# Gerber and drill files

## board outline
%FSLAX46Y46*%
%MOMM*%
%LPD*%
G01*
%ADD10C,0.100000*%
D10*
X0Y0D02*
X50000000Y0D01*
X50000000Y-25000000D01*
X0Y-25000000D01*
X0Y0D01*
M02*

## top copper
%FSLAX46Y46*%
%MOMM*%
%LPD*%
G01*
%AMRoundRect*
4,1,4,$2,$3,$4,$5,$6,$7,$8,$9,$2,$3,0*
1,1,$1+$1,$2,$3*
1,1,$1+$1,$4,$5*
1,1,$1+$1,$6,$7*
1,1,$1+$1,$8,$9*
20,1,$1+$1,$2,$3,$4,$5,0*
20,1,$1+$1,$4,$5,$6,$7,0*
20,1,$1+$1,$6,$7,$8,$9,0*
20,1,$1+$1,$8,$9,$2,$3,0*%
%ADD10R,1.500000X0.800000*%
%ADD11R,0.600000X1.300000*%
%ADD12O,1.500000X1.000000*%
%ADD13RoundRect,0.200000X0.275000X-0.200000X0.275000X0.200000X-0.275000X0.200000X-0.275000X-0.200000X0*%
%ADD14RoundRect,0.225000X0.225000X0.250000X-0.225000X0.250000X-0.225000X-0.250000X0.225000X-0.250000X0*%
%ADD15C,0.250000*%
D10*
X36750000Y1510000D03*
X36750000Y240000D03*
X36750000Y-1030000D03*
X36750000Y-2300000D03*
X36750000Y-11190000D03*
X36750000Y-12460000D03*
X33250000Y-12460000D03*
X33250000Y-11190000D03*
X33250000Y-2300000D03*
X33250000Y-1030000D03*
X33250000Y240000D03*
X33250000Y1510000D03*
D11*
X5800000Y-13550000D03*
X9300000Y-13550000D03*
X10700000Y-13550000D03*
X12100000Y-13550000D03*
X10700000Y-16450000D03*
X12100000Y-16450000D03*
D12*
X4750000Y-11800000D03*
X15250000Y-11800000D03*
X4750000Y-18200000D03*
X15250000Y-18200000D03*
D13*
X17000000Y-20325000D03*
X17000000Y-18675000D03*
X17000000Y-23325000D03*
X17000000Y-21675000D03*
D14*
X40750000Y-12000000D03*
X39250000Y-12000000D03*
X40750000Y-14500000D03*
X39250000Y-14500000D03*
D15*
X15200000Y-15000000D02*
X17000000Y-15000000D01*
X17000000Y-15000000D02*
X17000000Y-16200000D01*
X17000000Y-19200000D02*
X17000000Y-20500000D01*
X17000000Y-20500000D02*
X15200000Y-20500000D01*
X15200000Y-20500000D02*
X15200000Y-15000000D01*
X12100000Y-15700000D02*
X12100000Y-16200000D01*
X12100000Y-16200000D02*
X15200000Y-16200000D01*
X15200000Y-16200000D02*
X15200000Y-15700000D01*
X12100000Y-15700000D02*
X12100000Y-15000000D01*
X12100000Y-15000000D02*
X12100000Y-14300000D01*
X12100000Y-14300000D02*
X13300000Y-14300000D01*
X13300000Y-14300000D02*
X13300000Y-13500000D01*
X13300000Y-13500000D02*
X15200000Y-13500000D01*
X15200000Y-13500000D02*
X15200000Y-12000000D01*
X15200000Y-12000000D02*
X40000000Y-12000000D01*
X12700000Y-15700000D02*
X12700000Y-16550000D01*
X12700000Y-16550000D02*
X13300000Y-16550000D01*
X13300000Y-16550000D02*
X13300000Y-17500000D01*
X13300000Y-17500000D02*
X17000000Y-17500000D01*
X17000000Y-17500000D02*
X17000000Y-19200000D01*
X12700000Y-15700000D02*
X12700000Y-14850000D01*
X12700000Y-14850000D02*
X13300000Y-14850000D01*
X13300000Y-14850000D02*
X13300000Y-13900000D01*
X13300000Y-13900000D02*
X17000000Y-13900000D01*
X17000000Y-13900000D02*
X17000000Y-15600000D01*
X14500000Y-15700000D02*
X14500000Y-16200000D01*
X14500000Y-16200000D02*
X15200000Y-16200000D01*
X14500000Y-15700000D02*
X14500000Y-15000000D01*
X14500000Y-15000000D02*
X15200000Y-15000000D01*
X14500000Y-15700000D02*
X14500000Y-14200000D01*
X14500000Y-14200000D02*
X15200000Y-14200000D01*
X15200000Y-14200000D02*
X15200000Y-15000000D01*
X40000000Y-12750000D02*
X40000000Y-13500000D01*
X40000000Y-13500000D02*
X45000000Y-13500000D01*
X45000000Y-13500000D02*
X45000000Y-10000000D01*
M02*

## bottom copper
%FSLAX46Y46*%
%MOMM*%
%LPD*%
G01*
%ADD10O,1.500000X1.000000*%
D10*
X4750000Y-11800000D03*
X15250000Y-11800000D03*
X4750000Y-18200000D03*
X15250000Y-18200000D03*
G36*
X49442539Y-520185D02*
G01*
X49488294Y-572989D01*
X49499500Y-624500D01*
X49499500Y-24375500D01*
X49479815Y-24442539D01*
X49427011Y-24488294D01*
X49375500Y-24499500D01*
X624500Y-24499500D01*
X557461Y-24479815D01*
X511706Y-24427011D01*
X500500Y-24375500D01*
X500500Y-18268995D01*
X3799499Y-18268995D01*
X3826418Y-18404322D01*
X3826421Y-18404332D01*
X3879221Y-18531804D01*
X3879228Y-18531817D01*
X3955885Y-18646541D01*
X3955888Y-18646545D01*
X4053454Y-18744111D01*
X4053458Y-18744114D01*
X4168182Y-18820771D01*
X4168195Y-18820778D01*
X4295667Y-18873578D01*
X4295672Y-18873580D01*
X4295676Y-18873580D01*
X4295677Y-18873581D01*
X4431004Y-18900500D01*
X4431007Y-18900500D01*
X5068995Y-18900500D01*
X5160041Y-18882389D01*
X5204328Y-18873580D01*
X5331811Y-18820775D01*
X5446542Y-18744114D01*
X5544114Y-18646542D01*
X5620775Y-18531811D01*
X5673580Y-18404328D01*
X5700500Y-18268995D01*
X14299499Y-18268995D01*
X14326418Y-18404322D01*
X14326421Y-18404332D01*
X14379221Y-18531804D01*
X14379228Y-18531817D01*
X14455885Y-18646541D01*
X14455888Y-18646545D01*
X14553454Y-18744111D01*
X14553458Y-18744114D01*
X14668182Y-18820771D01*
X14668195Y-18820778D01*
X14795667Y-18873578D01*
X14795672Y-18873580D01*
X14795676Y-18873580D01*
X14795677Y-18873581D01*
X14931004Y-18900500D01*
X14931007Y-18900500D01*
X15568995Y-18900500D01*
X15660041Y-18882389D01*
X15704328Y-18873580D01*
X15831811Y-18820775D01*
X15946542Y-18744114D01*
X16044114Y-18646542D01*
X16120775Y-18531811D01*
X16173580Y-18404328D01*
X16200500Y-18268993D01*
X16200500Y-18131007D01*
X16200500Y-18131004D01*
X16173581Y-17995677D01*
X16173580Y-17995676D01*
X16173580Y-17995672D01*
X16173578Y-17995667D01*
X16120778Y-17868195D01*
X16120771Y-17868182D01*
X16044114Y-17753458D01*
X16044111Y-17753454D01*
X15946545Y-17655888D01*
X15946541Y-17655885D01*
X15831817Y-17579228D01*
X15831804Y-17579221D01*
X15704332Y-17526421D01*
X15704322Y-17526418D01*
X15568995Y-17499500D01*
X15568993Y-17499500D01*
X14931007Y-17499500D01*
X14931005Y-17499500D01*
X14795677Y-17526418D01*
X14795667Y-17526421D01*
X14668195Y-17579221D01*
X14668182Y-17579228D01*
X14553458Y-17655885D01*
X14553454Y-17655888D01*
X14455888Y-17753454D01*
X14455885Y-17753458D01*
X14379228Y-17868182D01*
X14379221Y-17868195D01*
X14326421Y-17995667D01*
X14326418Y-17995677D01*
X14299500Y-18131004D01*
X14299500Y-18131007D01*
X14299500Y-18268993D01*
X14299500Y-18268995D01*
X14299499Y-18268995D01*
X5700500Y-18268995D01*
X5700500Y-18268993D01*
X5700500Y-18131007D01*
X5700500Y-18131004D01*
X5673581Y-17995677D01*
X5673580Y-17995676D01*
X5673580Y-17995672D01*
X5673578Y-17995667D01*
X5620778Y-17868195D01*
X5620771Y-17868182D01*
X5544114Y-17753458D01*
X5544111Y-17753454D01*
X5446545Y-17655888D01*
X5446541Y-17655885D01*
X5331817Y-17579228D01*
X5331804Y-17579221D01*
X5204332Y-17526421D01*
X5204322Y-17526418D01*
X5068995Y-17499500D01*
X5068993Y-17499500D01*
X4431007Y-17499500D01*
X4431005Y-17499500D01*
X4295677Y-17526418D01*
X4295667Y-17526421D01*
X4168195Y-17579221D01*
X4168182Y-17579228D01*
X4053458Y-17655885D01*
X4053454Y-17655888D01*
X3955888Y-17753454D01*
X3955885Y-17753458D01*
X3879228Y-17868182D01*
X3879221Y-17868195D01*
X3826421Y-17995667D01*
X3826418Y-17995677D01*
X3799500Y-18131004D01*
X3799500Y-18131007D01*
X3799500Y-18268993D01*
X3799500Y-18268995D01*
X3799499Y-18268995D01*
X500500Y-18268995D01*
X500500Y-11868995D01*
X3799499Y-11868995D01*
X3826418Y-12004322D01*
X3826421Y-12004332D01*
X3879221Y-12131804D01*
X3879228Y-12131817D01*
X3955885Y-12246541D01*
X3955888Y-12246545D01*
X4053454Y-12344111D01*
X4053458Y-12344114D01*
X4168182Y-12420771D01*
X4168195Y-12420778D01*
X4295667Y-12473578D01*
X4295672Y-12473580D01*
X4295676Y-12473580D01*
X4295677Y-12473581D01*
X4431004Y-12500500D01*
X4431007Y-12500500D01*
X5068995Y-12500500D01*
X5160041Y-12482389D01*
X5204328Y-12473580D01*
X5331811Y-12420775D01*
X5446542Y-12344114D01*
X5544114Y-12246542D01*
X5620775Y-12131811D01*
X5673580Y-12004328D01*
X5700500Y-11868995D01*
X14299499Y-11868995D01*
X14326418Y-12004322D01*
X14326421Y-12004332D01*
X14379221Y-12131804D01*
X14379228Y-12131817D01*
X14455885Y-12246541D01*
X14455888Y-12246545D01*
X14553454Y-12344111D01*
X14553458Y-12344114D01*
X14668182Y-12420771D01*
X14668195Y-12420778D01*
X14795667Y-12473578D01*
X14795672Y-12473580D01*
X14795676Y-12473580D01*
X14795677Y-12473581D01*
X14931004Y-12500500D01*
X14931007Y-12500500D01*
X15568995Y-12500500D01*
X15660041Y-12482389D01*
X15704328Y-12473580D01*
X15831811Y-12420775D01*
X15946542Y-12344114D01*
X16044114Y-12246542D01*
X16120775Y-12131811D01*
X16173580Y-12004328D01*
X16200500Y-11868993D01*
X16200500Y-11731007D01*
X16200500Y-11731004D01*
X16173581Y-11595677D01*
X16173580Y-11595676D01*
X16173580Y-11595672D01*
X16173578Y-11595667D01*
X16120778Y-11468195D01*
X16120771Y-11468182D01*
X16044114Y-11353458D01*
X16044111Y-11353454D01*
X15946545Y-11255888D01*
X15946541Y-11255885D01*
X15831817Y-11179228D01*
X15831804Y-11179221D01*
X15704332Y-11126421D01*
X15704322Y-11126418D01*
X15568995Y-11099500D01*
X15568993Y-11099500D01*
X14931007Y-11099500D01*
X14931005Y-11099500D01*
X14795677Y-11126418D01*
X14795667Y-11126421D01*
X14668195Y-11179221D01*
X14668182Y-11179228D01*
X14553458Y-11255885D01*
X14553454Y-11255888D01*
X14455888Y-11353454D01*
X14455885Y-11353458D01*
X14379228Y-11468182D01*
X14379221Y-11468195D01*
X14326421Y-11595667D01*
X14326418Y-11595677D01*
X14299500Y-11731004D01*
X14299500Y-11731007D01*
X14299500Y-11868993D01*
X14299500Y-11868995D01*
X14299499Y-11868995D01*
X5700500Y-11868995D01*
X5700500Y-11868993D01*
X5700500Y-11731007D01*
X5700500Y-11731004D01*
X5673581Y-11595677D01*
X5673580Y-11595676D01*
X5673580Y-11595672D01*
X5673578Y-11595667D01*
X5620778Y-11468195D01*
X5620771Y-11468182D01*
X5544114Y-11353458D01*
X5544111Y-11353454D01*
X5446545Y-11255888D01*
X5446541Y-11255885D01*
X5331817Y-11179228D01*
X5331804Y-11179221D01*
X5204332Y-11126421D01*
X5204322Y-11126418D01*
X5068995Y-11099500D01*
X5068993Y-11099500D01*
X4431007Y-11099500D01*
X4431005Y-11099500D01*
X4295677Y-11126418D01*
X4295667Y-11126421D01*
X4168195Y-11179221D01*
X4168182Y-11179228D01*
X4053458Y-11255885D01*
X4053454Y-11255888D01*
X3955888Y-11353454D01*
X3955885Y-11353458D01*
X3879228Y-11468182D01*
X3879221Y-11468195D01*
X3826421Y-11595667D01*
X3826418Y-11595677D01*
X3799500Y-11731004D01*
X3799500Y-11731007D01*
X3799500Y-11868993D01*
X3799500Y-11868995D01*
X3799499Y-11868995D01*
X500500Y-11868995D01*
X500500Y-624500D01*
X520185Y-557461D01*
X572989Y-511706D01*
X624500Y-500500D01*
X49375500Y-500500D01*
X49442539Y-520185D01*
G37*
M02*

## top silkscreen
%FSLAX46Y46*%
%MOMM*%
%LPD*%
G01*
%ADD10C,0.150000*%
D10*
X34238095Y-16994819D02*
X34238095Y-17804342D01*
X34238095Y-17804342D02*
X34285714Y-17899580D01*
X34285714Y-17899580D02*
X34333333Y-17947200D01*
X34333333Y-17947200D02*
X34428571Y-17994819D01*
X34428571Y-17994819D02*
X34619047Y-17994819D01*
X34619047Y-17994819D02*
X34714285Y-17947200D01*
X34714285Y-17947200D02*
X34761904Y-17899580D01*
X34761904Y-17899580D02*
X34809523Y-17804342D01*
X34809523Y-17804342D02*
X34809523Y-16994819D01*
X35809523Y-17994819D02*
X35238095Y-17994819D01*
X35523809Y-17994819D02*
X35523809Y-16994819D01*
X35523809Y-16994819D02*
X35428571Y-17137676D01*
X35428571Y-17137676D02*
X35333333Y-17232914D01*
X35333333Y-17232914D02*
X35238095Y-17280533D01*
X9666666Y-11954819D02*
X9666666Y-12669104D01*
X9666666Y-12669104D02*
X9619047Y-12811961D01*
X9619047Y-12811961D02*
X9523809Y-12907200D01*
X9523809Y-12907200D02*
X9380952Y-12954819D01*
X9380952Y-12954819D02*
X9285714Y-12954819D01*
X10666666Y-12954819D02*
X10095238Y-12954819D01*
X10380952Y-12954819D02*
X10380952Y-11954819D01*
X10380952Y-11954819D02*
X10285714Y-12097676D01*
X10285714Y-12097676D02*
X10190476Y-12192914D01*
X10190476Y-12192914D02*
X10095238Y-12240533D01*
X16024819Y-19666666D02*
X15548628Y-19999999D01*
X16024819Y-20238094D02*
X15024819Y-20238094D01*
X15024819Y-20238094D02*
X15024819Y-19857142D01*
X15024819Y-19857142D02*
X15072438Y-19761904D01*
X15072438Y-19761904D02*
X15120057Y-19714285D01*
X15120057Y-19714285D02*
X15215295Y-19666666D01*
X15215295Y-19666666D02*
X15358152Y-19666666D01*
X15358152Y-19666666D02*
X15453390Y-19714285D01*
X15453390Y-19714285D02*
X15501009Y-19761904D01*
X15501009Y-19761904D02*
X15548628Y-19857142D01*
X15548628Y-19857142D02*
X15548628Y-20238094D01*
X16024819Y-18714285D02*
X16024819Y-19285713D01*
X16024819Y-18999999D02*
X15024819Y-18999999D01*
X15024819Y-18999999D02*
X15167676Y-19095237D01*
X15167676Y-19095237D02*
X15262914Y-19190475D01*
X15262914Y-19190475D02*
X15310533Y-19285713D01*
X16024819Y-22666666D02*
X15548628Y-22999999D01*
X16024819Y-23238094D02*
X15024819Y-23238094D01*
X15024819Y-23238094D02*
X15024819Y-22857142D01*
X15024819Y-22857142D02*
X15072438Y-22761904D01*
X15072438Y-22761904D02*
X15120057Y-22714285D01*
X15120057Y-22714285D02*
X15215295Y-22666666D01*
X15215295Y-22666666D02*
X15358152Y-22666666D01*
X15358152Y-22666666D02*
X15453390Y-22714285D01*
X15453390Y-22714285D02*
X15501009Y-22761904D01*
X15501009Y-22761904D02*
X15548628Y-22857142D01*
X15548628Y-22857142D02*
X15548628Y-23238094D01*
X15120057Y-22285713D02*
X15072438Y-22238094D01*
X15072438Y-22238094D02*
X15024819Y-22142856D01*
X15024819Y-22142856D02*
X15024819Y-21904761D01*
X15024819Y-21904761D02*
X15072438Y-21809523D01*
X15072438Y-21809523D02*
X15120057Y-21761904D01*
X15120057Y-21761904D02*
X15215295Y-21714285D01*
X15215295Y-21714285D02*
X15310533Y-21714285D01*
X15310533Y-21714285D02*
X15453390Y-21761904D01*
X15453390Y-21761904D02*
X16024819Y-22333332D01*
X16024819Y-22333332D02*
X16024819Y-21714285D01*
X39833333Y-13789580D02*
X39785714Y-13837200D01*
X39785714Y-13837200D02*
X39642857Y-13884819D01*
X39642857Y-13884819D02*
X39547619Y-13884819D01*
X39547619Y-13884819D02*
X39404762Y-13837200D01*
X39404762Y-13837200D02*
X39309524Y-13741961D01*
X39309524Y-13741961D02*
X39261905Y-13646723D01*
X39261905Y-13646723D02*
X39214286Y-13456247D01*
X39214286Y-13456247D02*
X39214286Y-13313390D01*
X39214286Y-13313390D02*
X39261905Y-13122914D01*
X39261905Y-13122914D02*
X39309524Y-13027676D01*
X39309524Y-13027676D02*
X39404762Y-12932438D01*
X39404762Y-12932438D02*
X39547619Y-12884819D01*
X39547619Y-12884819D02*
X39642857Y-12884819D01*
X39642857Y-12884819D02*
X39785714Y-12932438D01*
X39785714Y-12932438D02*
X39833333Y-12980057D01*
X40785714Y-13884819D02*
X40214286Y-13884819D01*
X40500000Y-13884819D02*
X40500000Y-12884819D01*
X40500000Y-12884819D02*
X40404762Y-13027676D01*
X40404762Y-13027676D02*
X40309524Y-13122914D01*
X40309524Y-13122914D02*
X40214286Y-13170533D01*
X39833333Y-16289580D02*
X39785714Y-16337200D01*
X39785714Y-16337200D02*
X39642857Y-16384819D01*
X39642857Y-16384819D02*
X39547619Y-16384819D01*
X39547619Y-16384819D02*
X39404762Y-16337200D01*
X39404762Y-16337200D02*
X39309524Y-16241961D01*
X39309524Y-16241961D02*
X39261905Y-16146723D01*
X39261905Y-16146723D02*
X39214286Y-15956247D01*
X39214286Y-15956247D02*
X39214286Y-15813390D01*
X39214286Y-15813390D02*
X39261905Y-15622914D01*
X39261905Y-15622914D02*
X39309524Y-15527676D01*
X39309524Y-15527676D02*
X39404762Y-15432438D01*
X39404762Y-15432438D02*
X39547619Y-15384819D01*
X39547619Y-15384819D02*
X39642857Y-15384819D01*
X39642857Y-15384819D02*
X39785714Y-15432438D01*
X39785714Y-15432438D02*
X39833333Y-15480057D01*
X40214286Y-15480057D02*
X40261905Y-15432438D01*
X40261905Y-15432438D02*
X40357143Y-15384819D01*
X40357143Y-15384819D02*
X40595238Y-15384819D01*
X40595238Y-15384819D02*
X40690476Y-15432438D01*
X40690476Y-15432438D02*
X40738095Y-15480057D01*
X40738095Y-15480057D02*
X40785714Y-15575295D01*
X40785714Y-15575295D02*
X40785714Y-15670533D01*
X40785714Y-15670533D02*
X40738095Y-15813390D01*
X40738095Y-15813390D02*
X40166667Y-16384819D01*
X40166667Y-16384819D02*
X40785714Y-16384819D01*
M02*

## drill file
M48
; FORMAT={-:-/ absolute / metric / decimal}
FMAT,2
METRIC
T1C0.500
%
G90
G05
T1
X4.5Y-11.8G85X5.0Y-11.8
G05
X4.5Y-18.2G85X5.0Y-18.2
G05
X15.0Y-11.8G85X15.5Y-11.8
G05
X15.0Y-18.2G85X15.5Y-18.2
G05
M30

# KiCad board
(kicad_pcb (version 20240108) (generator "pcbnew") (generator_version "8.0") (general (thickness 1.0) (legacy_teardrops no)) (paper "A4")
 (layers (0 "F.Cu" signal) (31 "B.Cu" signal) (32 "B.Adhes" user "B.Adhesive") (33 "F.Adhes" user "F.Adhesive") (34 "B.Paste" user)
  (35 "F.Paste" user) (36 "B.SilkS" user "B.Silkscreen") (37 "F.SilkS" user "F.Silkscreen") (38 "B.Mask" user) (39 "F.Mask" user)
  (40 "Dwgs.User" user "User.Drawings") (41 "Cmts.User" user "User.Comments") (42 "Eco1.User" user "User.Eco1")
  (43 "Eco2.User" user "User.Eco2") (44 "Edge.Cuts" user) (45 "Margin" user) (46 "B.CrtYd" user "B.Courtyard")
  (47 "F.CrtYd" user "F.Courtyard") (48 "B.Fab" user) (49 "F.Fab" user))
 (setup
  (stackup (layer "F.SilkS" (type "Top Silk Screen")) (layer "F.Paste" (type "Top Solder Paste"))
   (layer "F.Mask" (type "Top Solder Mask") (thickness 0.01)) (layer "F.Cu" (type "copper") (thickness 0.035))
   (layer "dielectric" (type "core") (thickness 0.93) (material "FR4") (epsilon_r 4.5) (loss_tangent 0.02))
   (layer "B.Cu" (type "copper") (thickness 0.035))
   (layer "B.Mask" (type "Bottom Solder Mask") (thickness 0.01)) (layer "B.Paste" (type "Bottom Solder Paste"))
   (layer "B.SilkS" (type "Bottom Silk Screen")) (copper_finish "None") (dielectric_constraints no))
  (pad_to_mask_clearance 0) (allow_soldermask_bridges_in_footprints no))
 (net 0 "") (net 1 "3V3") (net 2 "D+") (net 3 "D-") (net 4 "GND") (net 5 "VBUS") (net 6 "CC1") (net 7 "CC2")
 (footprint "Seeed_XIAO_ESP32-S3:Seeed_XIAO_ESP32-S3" (layer "F.Cu") (at 35 15 180)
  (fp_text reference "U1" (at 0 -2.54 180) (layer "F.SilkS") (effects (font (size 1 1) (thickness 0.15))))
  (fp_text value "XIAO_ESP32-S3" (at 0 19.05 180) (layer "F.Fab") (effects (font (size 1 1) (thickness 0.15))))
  (pad "1" smd rect (at -1.75 16.51 180) (size 1.5 0.8) (layers "F.Cu" "F.Paste" "F.Mask") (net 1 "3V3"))
  (pad "2" smd rect (at -1.75 15.24 180) (size 1.5 0.8) (layers "F.Cu" "F.Paste" "F.Mask") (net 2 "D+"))
  (pad "3" smd rect (at -1.75 13.97 180) (size 1.5 0.8) (layers "F.Cu" "F.Paste" "F.Mask") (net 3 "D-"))
  (pad "4" smd rect (at -1.75 12.7 180) (size 1.5 0.8) (layers "F.Cu" "F.Paste" "F.Mask") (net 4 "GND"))
  (pad "5" smd rect (at -1.75 3.81 180) (size 1.5 0.8) (layers "F.Cu" "F.Paste" "F.Mask") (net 4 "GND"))
  (pad "6" smd rect (at -1.75 2.54 180) (size 1.5 0.8) (layers "F.Cu" "F.Paste" "F.Mask") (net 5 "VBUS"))
  (pad "7" smd rect (at 1.75 2.54 180) (size 1.5 0.8) (layers "F.Cu" "F.Paste" "F.Mask") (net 4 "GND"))
  (pad "8" smd rect (at 1.75 3.81 180) (size 1.5 0.8) (layers "F.Cu" "F.Paste" "F.Mask") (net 4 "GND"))
  (pad "9" smd rect (at 1.75 12.7 180) (size 1.5 0.8) (layers "F.Cu" "F.Paste" "F.Mask") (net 4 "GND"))
  (pad "10" smd rect (at 1.75 13.97 180) (size 1.5 0.8) (layers "F.Cu" "F.Paste" "F.Mask") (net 3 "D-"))
  (pad "11" smd rect (at 1.75 15.24 180) (size 1.5 0.8) (layers "F.Cu" "F.Paste" "F.Mask") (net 2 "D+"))
  (pad "12" smd rect (at 1.75 16.51 180) (size 1.5 0.8) (layers "F.Cu" "F.Paste" "F.Mask") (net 1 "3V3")))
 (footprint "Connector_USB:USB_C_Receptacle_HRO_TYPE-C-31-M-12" (layer "F.Cu") (at 10 15 0)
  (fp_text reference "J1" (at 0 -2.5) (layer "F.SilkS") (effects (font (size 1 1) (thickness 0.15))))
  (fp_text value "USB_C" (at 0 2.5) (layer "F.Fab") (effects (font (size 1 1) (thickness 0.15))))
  (pad "A1" smd rect (at -4.2 -1.45) (size 0.6 1.3) (layers "F.Cu" "F.Paste" "F.Mask") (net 4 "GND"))
  (pad "A4" smd rect (at -0.7 -1.45) (size 0.6 1.3) (layers "F.Cu" "F.Paste" "F.Mask") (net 5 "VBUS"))
  (pad "A6" smd rect (at 0.7 -1.45) (size 0.6 1.3) (layers "F.Cu" "F.Paste" "F.Mask") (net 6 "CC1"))
  (pad "A7" smd rect (at 2.1 -1.45) (size 0.6 1.3) (layers "F.Cu" "F.Paste" "F.Mask") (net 2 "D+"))
  (pad "B6" smd rect (at 0.7 1.45) (size 0.6 1.3) (layers "F.Cu" "F.Paste" "F.Mask") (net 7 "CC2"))
  (pad "B7" smd rect (at 2.1 1.45) (size 0.6 1.3) (layers "F.Cu" "F.Paste" "F.Mask") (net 3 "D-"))
  (pad "S1" thru_hole oval (at -5.25 -3.2) (size 1.5 1) (drill oval 1 0.5) (layers "*.Cu" "*.Mask"))
  (pad "S2" thru_hole oval (at 5.25 -3.2) (size 1.5 1) (drill oval 1 0.5) (layers "*.Cu" "*.Mask"))
  (pad "S3" thru_hole oval (at -5.25 3.2) (size 1.5 1) (drill oval 1 0.5) (layers "*.Cu" "*.Mask"))
  (pad "S4" thru_hole oval (at 5.25 3.2) (size 1.5 1) (drill oval 1 0.5) (layers "*.Cu" "*.Mask")))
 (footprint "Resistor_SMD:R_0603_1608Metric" (layer "F.Cu") (at 17 19.5 90)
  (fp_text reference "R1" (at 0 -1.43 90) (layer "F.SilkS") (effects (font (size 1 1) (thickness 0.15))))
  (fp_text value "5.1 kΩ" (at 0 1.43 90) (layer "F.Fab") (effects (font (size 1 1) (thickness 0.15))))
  (pad "1" smd roundrect (at -0.825 0 90) (size 0.8 0.95) (layers "F.Cu" "F.Paste" "F.Mask") (roundrect_rratio 0.25) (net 6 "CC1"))
  (pad "2" smd roundrect (at 0.825 0 90) (size 0.8 0.95) (layers "F.Cu" "F.Paste" "F.Mask") (roundrect_rratio 0.25) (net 4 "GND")))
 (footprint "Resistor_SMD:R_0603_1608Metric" (layer "F.Cu") (at 17 22.5 90)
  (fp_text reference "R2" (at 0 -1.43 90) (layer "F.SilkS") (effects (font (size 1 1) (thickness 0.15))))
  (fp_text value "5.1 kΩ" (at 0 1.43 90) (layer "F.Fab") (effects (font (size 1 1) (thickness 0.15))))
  (pad "1" smd roundrect (at -0.825 0 90) (size 0.8 0.95) (layers "F.Cu" "F.Paste" "F.Mask") (roundrect_rratio 0.25) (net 7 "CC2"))
  (pad "2" smd roundrect (at 0.825 0 90) (size 0.8 0.95) (layers "F.Cu" "F.Paste" "F.Mask") (roundrect_rratio 0.25) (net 4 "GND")))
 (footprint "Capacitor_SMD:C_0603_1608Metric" (layer "F.Cu") (at 40 12 180)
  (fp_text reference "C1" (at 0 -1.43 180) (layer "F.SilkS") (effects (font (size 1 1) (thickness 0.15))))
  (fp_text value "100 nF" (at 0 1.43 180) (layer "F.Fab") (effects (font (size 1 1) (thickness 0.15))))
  (pad "1" smd roundrect (at -0.75 0 180) (size 0.9 0.95) (layers "F.Cu" "F.Paste" "F.Mask") (roundrect_rratio 0.25) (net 1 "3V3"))
  (pad "2" smd roundrect (at 0.75 0 180) (size 0.9 0.95) (layers "F.Cu" "F.Paste" "F.Mask") (roundrect_rratio 0.25) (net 4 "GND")))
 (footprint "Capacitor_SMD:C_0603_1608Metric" (layer "F.Cu") (at 40 14.5 180)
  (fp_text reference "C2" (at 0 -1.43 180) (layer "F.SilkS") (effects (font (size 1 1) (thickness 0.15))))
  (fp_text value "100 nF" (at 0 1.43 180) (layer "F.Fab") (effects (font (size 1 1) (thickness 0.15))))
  (pad "1" smd roundrect (at -0.75 0 180) (size 0.9 0.95) (layers "F.Cu" "F.Paste" "F.Mask") (roundrect_rratio 0.25) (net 5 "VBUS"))
  (pad "2" smd roundrect (at 0.75 0 180) (size 0.9 0.95) (layers "F.Cu" "F.Paste" "F.Mask") (roundrect_rratio 0.25) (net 4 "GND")))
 (gr_rect (start 0 0) (end 50 25) (stroke (width 0.1) (type default)) (fill none) (layer "Edge.Cuts"))
 (segment (start 15.2 15) (end 17 15) (width 0.25) (layer "F.Cu") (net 4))
 (segment (start 17 15) (end 17 16.2) (width 0.25) (layer "F.Cu") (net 4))
 (segment (start 17 19.2) (end 17 20.5) (width 0.25) (layer "F.Cu") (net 4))
 (segment (start 17 20.5) (end 15.2 20.5) (width 0.25) (layer "F.Cu") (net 4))
 (segment (start 15.2 20.5) (end 15.2 15) (width 0.25) (layer "F.Cu") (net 4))
 (segment (start 12.1 15.7) (end 12.1 16.2) (width 0.25) (layer "F.Cu") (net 5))
 (segment (start 12.1 16.2) (end 15.2 16.2) (width 0.25) (layer "F.Cu") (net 5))
 (segment (start 15.2 16.2) (end 15.2 15.7) (width 0.25) (layer "F.Cu") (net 5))
 (segment (start 12.1 15.7) (end 12.1 15) (width 0.25) (layer "F.Cu") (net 5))
 (segment (start 12.1 15) (end 12.1 14.3) (width 0.25) (layer "F.Cu") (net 5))
 (segment (start 12.1 14.3) (end 13.3 14.3) (width 0.25) (layer "F.Cu") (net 5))
 (segment (start 13.3 14.3) (end 13.3 13.5) (width 0.25) (layer "F.Cu") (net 5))
 (segment (start 13.3 13.5) (end 15.2 13.5) (width 0.25) (layer "F.Cu") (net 5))
 (segment (start 15.2 13.5) (end 15.2 12) (width 0.25) (layer "F.Cu") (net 5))
 (segment (start 15.2 12) (end 40 12) (width 0.25) (layer "F.Cu") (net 5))
 (segment (start 12.7 15.7) (end 12.7 16.55) (width 0.25) (layer "F.Cu") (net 6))
 (segment (start 12.7 16.55) (end 13.3 16.55) (width 0.25) (layer "F.Cu") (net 6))
 (segment (start 13.3 16.55) (end 13.3 17.5) (width 0.25) (layer "F.Cu") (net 6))
 (segment (start 13.3 17.5) (end 17 17.5) (width 0.25) (layer "F.Cu") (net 6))
 (segment (start 17 17.5) (end 17 19.2) (width 0.25) (layer "F.Cu") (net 6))
 (segment (start 12.7 15.7) (end 12.7 14.85) (width 0.25) (layer "F.Cu") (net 7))
 (segment (start 12.7 14.85) (end 13.3 14.85) (width 0.25) (layer "F.Cu") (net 7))
 (segment (start 13.3 14.85) (end 13.3 13.9) (width 0.25) (layer "F.Cu") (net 7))
 (segment (start 13.3 13.9) (end 17 13.9) (width 0.25) (layer "F.Cu") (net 7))
 (segment (start 17 13.9) (end 17 15.6) (width 0.25) (layer "F.Cu") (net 7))
 (segment (start 14.5 15.7) (end 14.5 16.2) (width 0.25) (layer "F.Cu") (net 2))
 (segment (start 14.5 16.2) (end 15.2 16.2) (width 0.25) (layer "F.Cu") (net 2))
 (segment (start 14.5 15.7) (end 14.5 15) (width 0.25) (layer "F.Cu") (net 2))
 (segment (start 14.5 15) (end 15.2 15) (width 0.25) (layer "F.Cu") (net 2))
 (segment (start 14.5 15.7) (end 14.5 14.2) (width 0.25) (layer "F.Cu") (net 3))
 (segment (start 14.5 14.2) (end 15.2 14.2) (width 0.25) (layer "F.Cu") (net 3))
 (segment (start 15.2 14.2) (end 15.2 15) (width 0.25) (layer "F.Cu") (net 3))
 (segment (start 40 12.75) (end 40 13.5) (width 0.25) (layer "F.Cu") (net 1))
 (segment (start 40 13.5) (end 45 13.5) (width 0.25) (layer "F.Cu") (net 1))
 (segment (start 45 13.5) (end 45 10) (width 0.25) (layer "F.Cu") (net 1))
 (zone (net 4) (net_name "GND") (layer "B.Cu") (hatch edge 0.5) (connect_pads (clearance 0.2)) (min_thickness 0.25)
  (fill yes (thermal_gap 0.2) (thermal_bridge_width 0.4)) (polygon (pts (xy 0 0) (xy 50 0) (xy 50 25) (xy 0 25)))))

